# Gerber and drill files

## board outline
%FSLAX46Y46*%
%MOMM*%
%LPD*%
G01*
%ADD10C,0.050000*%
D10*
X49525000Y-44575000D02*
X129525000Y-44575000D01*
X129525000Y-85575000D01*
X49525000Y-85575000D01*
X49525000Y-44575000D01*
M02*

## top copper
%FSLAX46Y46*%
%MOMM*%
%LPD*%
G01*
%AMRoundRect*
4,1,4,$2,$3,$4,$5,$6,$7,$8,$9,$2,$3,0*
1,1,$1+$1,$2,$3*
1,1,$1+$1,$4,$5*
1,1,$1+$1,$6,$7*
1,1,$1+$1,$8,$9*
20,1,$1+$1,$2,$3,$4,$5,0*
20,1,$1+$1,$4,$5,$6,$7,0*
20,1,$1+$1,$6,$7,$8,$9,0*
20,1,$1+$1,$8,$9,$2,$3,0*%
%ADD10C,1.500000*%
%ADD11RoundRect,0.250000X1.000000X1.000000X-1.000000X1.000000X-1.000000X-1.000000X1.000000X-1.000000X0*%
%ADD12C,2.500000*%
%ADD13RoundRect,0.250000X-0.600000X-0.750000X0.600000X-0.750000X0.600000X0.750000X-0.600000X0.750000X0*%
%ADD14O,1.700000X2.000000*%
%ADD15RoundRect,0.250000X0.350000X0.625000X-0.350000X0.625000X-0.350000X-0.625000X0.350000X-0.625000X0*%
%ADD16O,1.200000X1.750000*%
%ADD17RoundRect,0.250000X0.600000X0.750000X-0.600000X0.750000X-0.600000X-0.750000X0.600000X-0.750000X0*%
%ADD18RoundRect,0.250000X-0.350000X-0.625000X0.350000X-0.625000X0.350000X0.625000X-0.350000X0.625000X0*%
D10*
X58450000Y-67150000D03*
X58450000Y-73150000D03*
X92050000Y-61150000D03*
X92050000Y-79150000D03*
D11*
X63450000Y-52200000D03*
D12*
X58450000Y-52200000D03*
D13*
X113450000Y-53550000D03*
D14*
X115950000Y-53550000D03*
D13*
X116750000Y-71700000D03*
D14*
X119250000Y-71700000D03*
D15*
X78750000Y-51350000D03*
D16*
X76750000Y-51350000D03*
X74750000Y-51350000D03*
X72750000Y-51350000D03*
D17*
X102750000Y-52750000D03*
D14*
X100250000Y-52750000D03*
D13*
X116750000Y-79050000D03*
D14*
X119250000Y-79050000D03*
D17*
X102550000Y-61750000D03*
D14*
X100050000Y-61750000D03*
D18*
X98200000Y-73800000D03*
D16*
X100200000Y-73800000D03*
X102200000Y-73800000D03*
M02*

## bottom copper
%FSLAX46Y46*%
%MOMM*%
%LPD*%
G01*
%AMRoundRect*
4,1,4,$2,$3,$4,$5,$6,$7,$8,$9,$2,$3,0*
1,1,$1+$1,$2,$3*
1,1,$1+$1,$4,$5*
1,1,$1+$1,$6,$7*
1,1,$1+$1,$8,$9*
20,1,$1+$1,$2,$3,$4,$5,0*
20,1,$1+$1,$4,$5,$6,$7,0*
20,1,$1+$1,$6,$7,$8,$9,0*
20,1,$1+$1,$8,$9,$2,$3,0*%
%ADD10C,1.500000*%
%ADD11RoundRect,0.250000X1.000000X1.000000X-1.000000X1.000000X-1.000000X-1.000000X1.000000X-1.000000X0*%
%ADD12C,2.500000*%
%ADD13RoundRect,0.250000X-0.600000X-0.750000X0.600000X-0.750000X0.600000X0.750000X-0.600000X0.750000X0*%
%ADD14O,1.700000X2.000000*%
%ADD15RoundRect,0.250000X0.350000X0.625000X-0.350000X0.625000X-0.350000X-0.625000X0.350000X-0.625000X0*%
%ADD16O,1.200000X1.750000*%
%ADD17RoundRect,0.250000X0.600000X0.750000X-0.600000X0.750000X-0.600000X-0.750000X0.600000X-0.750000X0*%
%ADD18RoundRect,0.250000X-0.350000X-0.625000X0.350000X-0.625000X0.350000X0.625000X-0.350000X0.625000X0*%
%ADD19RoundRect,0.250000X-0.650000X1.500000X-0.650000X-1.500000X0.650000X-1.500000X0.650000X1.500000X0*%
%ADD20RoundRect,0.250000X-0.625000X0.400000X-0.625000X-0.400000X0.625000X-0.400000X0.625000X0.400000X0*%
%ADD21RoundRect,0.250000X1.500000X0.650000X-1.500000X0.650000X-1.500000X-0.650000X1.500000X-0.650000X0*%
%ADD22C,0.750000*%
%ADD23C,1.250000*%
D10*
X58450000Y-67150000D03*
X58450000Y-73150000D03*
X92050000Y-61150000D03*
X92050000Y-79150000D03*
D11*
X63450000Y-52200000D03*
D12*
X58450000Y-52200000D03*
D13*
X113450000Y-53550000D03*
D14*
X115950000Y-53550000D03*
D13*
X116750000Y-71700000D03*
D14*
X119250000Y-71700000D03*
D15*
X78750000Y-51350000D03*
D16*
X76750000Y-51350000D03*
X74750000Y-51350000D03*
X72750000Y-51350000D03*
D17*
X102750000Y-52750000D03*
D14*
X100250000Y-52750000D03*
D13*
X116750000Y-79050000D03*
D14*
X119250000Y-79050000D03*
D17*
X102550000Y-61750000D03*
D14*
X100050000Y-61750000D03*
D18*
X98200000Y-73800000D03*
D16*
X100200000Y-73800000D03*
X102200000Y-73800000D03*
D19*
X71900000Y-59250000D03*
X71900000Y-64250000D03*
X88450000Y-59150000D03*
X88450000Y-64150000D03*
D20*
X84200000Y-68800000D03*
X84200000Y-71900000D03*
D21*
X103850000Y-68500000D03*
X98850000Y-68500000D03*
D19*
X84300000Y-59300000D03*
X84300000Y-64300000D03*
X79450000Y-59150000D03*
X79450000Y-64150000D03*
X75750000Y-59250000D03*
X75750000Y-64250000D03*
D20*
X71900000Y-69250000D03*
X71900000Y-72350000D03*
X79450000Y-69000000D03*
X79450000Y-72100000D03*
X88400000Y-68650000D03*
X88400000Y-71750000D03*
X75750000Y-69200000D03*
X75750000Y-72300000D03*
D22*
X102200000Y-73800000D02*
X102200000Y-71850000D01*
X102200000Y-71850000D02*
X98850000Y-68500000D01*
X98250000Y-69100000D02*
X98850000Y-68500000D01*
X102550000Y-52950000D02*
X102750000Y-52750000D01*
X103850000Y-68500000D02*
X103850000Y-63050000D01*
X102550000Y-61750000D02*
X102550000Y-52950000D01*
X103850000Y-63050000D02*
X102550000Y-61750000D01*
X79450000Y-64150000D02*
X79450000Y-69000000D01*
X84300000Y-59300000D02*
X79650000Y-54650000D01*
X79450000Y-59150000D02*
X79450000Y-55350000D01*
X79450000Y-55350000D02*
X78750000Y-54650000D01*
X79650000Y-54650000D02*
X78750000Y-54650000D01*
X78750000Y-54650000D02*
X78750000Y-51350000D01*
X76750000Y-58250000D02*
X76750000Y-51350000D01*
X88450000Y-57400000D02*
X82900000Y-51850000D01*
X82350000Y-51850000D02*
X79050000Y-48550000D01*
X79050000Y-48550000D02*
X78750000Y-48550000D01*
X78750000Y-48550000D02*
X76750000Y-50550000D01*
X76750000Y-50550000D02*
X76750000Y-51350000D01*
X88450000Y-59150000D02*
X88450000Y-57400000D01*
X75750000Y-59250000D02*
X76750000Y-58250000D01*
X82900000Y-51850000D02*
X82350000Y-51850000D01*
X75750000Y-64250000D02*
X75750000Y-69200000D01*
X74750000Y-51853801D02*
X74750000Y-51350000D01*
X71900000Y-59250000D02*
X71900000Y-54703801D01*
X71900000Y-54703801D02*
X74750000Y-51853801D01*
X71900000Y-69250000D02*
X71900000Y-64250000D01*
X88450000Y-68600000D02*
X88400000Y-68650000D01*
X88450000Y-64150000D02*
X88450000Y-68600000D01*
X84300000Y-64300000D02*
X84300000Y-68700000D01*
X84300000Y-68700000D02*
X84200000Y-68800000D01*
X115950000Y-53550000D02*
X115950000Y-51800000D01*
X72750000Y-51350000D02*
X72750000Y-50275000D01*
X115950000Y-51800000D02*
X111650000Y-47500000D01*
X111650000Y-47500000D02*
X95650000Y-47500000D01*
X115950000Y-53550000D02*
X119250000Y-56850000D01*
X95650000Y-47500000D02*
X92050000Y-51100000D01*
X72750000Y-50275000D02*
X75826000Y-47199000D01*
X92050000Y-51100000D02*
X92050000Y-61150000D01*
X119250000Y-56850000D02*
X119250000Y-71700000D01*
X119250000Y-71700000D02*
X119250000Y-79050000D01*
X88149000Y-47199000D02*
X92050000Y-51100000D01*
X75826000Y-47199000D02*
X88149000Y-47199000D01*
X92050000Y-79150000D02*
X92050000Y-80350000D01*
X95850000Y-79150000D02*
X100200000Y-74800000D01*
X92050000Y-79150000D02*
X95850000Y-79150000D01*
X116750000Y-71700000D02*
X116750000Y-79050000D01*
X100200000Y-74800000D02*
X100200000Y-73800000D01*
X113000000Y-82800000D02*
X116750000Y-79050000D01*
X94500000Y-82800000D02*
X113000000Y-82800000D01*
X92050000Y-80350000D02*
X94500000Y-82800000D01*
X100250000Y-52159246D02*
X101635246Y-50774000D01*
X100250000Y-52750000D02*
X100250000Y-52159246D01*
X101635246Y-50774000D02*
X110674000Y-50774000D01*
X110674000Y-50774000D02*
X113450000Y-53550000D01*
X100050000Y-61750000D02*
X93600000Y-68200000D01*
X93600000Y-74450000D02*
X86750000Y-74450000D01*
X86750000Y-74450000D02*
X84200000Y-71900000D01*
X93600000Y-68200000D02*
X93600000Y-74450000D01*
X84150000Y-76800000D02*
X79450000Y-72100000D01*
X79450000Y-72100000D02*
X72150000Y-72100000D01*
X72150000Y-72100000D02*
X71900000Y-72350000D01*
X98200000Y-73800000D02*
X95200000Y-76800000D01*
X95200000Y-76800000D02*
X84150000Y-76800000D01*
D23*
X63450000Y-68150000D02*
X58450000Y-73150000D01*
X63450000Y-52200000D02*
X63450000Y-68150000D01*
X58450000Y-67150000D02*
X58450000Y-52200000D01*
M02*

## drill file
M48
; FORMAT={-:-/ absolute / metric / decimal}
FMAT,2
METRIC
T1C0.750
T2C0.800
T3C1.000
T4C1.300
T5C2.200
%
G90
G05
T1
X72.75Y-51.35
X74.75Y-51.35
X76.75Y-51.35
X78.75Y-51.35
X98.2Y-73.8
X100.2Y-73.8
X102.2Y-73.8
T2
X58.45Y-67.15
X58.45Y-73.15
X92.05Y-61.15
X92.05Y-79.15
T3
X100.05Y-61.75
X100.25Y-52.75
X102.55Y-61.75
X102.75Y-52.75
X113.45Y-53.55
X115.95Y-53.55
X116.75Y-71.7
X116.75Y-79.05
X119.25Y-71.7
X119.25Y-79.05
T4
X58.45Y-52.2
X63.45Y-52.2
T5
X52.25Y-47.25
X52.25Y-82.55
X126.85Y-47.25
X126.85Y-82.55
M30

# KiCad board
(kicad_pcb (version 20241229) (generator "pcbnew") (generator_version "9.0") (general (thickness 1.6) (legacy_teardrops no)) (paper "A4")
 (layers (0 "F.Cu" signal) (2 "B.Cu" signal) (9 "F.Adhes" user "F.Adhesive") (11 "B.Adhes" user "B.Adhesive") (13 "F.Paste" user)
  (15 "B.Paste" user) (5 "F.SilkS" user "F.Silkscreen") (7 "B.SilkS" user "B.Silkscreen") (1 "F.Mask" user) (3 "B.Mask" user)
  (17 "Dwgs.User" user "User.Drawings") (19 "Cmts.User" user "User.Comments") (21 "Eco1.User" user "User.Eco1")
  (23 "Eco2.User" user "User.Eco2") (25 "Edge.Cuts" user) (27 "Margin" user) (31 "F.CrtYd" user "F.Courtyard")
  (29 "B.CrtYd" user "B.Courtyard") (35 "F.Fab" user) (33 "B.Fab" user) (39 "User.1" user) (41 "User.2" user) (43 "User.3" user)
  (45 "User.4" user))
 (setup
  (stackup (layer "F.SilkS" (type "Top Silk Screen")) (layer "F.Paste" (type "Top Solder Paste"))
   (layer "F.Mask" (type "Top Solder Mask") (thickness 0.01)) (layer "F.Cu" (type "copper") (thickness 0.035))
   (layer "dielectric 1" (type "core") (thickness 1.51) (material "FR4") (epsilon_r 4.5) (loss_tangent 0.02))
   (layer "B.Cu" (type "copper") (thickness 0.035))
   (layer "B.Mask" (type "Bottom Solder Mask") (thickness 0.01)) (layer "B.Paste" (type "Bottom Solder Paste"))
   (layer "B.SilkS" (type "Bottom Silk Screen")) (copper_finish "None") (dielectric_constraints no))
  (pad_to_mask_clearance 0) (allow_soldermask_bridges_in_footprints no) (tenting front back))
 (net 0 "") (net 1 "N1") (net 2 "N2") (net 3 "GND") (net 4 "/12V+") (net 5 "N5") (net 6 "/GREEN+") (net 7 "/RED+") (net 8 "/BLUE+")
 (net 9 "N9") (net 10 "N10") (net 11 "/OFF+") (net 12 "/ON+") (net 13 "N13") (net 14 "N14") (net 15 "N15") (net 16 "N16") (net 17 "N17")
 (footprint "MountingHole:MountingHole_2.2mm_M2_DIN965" (layer "F.Cu") (at 52.25 47.25)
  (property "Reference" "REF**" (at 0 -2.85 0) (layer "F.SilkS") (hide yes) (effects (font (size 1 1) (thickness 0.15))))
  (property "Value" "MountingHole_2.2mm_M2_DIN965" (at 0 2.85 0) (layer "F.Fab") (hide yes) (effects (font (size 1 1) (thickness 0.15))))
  (pad "" np_thru_hole circle (at 0 0) (size 2.2 2.2) (drill 2.2) (layers "*.Cu" "*.Mask")))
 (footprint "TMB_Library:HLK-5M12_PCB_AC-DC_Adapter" (layer "F.Cu") (at 75.25 70.15)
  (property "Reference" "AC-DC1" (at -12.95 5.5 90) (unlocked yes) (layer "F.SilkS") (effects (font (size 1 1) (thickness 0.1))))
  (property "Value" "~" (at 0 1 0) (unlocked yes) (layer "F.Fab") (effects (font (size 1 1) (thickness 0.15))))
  (pad "1" thru_hole circle (at -16.8 -3) (size 1.5 1.5) (drill 0.8) (layers "*.Cu" "*.Mask") (remove_unused_layers yes)
   (keep_end_layers yes) (zone_layer_connections) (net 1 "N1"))
  (pad "2" thru_hole circle (at -16.8 3) (size 1.5 1.5) (drill 0.8) (layers "*.Cu" "*.Mask") (remove_unused_layers yes)
   (keep_end_layers yes) (zone_layer_connections) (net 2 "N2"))
  (pad "3" thru_hole circle (at 16.8 -9) (size 1.5 1.5) (drill 0.8) (layers "*.Cu" "*.Mask") (remove_unused_layers yes)
   (keep_end_layers yes) (zone_layer_connections) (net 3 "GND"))
  (pad "4" thru_hole circle (at 16.8 9) (size 1.5 1.5) (drill 0.8) (layers "*.Cu" "*.Mask") (remove_unused_layers yes) (keep_end_layers yes)
   (zone_layer_connections) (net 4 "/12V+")))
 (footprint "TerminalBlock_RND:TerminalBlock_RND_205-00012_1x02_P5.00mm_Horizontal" (layer "F.Cu") (at 63.45 52.2 180)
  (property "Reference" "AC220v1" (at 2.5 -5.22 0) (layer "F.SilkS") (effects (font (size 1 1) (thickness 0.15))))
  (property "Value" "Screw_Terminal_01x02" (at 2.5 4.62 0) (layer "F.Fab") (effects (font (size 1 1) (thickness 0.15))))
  (pad "1" thru_hole roundrect (at 0 0 180) (size 2.5 2.5) (drill 1.3) (layers "*.Cu" "*.Mask") (remove_unused_layers no)
   (roundrect_rratio 0.1) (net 2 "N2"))
  (pad "2" thru_hole circle (at 5 0 180) (size 2.5 2.5) (drill 1.3) (layers "*.Cu" "*.Mask") (remove_unused_layers no) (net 1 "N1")))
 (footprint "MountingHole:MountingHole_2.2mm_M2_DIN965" (layer "F.Cu") (at 52.25 82.55)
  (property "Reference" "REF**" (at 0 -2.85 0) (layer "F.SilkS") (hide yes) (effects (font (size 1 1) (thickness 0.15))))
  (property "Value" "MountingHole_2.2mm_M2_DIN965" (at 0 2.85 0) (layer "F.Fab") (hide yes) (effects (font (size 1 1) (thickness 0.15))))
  (pad "" np_thru_hole circle (at 0 0) (size 2.2 2.2) (drill 2.2) (layers "*.Cu" "*.Mask")))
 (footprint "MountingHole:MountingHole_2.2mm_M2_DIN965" (layer "F.Cu") (at 126.85 82.55)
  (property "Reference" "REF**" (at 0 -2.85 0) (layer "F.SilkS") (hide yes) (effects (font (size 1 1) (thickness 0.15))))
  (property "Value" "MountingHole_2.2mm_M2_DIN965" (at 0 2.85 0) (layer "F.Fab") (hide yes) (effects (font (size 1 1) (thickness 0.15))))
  (pad "" np_thru_hole circle (at 0 0) (size 2.2 2.2) (drill 2.2) (layers "*.Cu" "*.Mask")))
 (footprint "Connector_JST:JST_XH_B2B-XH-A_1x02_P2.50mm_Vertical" (layer "F.Cu") (at 113.45 53.55)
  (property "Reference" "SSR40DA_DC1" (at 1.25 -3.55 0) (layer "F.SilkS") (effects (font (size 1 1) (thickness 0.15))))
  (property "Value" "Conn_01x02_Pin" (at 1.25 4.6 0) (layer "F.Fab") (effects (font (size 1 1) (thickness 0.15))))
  (pad "1" thru_hole roundrect (at 0 0) (size 1.7 2) (drill 1) (layers "*.Cu" "*.Mask") (remove_unused_layers no)
   (roundrect_rratio 0.147059) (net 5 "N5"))
  (pad "2" thru_hole oval (at 2.5 0) (size 1.7 2) (drill 1) (layers "*.Cu" "*.Mask") (remove_unused_layers no) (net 3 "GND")))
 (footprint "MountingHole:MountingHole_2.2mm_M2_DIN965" (layer "F.Cu") (at 126.85 47.25)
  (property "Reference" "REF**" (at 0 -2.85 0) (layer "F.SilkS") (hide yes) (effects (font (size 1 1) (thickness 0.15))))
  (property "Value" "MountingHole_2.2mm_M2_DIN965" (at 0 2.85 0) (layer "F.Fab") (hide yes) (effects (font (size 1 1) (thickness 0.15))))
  (pad "" np_thru_hole circle (at 0 0) (size 2.2 2.2) (drill 2.2) (layers "*.Cu" "*.Mask")))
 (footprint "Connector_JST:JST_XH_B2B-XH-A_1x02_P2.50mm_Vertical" (layer "F.Cu") (at 116.75 71.7)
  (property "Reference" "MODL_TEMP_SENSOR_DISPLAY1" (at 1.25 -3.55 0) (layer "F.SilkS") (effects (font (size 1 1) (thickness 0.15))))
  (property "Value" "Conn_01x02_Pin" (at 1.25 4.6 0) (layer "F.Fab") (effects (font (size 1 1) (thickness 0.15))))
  (pad "1" thru_hole roundrect (at 0 0) (size 1.7 2) (drill 1) (layers "*.Cu" "*.Mask") (remove_unused_layers no)
   (roundrect_rratio 0.147059) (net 4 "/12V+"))
  (pad "2" thru_hole oval (at 2.5 0) (size 1.7 2) (drill 1) (layers "*.Cu" "*.Mask") (remove_unused_layers no) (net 3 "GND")))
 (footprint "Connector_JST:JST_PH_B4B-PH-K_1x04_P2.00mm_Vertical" (layer "F.Cu") (at 78.75 51.35 180)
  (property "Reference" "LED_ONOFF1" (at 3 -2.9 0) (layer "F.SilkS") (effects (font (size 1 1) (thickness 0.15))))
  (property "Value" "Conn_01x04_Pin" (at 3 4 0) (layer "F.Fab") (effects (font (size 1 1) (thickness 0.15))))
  (pad "1" thru_hole roundrect (at 0 0 180) (size 1.2 1.75) (drill 0.75) (layers "*.Cu" "*.Mask") (remove_unused_layers no)
   (roundrect_rratio 0.208333) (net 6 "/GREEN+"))
  (pad "2" thru_hole oval (at 2 0 180) (size 1.2 1.75) (drill 0.75) (layers "*.Cu" "*.Mask") (remove_unused_layers no) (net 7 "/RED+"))
  (pad "3" thru_hole oval (at 4 0 180) (size 1.2 1.75) (drill 0.75) (layers "*.Cu" "*.Mask") (remove_unused_layers no) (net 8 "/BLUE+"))
  (pad "4" thru_hole oval (at 6 0 180) (size 1.2 1.75) (drill 0.75) (layers "*.Cu" "*.Mask") (remove_unused_layers no) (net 3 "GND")))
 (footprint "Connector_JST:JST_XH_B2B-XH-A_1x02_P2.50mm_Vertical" (layer "F.Cu") (at 102.75 52.75 180)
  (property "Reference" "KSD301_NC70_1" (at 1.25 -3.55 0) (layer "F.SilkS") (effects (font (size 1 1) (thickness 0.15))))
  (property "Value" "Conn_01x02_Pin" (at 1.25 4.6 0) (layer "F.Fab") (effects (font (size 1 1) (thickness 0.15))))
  (pad "1" thru_hole roundrect (at 0 0 180) (size 1.7 2) (drill 1) (layers "*.Cu" "*.Mask") (remove_unused_layers no)
   (roundrect_rratio 0.147059) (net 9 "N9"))
  (pad "2" thru_hole oval (at 2.5 0 180) (size 1.7 2) (drill 1) (layers "*.Cu" "*.Mask") (remove_unused_layers no) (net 5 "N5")))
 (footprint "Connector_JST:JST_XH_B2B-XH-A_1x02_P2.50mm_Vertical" (layer "F.Cu") (at 116.75 79.05)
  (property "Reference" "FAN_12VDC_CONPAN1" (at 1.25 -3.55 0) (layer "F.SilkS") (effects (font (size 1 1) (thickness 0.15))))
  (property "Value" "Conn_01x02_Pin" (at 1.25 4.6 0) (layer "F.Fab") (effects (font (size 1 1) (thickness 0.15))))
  (pad "1" thru_hole roundrect (at 0 0) (size 1.7 2) (drill 1) (layers "*.Cu" "*.Mask") (remove_unused_layers no)
   (roundrect_rratio 0.147059) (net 4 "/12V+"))
  (pad "2" thru_hole oval (at 2.5 0) (size 1.7 2) (drill 1) (layers "*.Cu" "*.Mask") (remove_unused_layers no) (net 3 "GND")))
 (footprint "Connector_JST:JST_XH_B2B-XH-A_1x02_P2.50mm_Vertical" (layer "F.Cu") (at 102.55 61.75 180)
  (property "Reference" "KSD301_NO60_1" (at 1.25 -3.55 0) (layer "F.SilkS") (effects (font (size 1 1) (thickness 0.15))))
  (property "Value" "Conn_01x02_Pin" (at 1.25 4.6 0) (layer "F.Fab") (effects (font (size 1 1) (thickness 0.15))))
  (pad "1" thru_hole roundrect (at 0 0 180) (size 1.7 2) (drill 1) (layers "*.Cu" "*.Mask") (remove_unused_layers no)
   (roundrect_rratio 0.147059) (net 9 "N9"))
  (pad "2" thru_hole oval (at 2.5 0 180) (size 1.7 2) (drill 1) (layers "*.Cu" "*.Mask") (remove_unused_layers no) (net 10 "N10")))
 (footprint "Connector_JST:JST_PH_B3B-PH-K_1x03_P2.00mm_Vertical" (layer "F.Cu") (at 98.2 73.8)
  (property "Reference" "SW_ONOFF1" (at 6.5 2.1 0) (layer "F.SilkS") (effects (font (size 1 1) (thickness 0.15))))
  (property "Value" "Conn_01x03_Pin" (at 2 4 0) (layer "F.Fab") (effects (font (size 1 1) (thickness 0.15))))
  (pad "1" thru_hole roundrect (at 0 0) (size 1.2 1.75) (drill 0.75) (layers "*.Cu" "*.Mask") (remove_unused_layers no)
   (roundrect_rratio 0.208333) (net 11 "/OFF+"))
  (pad "2" thru_hole oval (at 2 0) (size 1.2 1.75) (drill 0.75) (layers "*.Cu" "*.Mask") (remove_unused_layers no) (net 4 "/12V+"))
  (pad "3" thru_hole oval (at 4 0) (size 1.2 1.75) (drill 0.75) (layers "*.Cu" "*.Mask") (remove_unused_layers no) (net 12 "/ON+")))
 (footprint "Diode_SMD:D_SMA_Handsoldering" (layer "B.Cu") (at 71.9 61.75 -90)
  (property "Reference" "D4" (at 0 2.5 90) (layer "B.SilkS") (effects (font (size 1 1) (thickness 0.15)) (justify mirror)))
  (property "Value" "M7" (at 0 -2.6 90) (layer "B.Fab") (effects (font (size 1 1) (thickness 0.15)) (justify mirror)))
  (pad "1" smd roundrect (at -2.5 0 270) (size 3.5 1.8) (layers "B.Cu" "B.Mask" "B.Paste") (roundrect_rratio 0.1388888889) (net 8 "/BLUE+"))
  (pad "2" smd roundrect (at 2.5 0 270) (size 3.5 1.8) (layers "B.Cu" "B.Mask" "B.Paste") (roundrect_rratio 0.1388888889) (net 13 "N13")))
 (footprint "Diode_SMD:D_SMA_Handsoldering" (layer "B.Cu") (at 88.45 61.65 -90)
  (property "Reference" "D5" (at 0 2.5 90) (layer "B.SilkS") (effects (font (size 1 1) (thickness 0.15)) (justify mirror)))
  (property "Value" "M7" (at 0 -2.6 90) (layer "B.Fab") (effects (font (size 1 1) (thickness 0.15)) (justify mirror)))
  (pad "1" smd roundrect (at -2.5 0 270) (size 3.5 1.8) (layers "B.Cu" "B.Mask" "B.Paste") (roundrect_rratio 0.1388888889) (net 7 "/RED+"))
  (pad "2" smd roundrect (at 2.5 0 270) (size 3.5 1.8) (layers "B.Cu" "B.Mask" "B.Paste") (roundrect_rratio 0.1388888889) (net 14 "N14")))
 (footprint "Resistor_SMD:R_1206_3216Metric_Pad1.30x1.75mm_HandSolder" (layer "B.Cu") (at 84.2 70.35 -90)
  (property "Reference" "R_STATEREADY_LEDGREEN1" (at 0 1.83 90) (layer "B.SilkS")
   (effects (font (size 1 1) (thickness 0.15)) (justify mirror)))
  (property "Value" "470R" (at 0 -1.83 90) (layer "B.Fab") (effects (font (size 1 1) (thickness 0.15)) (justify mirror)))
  (pad "1" smd roundrect (at -1.55 0 270) (size 1.3 1.75) (layers "B.Cu" "B.Mask" "B.Paste") (roundrect_rratio 0.192308) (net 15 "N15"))
  (pad "2" smd roundrect (at 1.55 0 270) (size 1.3 1.75) (layers "B.Cu" "B.Mask" "B.Paste") (roundrect_rratio 0.192308) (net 10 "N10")))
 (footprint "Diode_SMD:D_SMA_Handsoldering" (layer "B.Cu") (at 101.35 68.5 180)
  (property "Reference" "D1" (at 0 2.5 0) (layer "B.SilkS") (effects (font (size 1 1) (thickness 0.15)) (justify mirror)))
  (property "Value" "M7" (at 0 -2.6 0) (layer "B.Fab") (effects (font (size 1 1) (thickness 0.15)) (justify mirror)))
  (pad "1" smd roundrect (at -2.5 0 180) (size 3.5 1.8) (layers "B.Cu" "B.Mask" "B.Paste") (roundrect_rratio 0.1388888889) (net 9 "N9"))
  (pad "2" smd roundrect (at 2.5 0 180) (size 3.5 1.8) (layers "B.Cu" "B.Mask" "B.Paste") (roundrect_rratio 0.1388888889) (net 12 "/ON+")))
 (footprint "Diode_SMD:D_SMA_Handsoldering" (layer "B.Cu") (at 84.3 61.8 -90)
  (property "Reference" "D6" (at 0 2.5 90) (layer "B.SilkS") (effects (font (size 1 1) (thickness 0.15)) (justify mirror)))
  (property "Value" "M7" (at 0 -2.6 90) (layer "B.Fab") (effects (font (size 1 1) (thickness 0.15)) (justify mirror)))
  (pad "1" smd roundrect (at -2.5 0 270) (size 3.5 1.8) (layers "B.Cu" "B.Mask" "B.Paste") (roundrect_rratio 0.1388888889) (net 6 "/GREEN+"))
  (pad "2" smd roundrect (at 2.5 0 270) (size 3.5 1.8) (layers "B.Cu" "B.Mask" "B.Paste") (roundrect_rratio 0.1388888889) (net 15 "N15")))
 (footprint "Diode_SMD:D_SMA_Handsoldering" (layer "B.Cu") (at 79.45 61.65 -90)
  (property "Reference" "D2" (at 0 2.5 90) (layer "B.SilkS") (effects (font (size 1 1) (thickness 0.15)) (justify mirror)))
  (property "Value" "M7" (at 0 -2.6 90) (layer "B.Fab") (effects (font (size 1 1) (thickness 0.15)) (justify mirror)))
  (pad "1" smd roundrect (at -2.5 0 270) (size 3.5 1.8) (layers "B.Cu" "B.Mask" "B.Paste") (roundrect_rratio 0.1388888889) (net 6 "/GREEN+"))
  (pad "2" smd roundrect (at 2.5 0 270) (size 3.5 1.8) (layers "B.Cu" "B.Mask" "B.Paste") (roundrect_rratio 0.1388888889) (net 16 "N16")))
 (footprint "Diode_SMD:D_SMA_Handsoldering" (layer "B.Cu") (at 75.75 61.75 -90)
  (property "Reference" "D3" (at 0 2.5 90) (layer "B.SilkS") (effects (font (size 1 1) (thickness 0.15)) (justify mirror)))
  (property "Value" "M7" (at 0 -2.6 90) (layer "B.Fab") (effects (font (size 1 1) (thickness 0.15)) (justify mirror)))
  (pad "1" smd roundrect (at -2.5 0 270) (size 3.5 1.8) (layers "B.Cu" "B.Mask" "B.Paste") (roundrect_rratio 0.1388888889) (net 7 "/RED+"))
  (pad "2" smd roundrect (at 2.5 0 270) (size 3.5 1.8) (layers "B.Cu" "B.Mask" "B.Paste") (roundrect_rratio 0.1388888889) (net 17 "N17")))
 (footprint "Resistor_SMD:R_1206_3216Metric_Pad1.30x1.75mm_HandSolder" (layer "B.Cu") (at 71.9 70.8 -90)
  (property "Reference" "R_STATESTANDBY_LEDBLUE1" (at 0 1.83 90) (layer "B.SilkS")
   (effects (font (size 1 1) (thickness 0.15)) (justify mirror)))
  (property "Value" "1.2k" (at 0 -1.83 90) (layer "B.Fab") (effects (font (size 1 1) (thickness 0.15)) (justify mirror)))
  (pad "1" smd roundrect (at -1.55 0 270) (size 1.3 1.75) (layers "B.Cu" "B.Mask" "B.Paste") (roundrect_rratio 0.192308) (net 13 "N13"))
  (pad "2" smd roundrect (at 1.55 0 270) (size 1.3 1.75) (layers "B.Cu" "B.Mask" "B.Paste") (roundrect_rratio 0.192308) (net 11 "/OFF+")))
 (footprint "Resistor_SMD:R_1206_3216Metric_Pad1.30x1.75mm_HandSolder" (layer "B.Cu") (at 79.45 70.55 -90)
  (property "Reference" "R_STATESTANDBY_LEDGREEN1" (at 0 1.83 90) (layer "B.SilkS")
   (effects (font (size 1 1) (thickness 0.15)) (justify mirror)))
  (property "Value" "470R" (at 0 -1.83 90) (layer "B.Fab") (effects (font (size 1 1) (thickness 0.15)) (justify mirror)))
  (pad "1" smd roundrect (at -1.55 0 270) (size 1.3 1.75) (layers "B.Cu" "B.Mask" "B.Paste") (roundrect_rratio 0.192308) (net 16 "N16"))
  (pad "2" smd roundrect (at 1.55 0 270) (size 1.3 1.75) (layers "B.Cu" "B.Mask" "B.Paste") (roundrect_rratio 0.192308) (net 11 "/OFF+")))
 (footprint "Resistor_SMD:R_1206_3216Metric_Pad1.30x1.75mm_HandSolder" (layer "B.Cu") (at 88.4 70.2 -90)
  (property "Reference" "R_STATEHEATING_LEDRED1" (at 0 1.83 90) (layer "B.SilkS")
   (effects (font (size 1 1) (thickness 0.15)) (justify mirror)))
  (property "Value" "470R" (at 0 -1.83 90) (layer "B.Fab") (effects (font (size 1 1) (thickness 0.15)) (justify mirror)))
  (pad "1" smd roundrect (at -1.55 0 270) (size 1.3 1.75) (layers "B.Cu" "B.Mask" "B.Paste") (roundrect_rratio 0.192308) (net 14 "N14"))
  (pad "2" smd roundrect (at 1.55 0 270) (size 1.3 1.75) (layers "B.Cu" "B.Mask" "B.Paste") (roundrect_rratio 0.192308) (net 5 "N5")))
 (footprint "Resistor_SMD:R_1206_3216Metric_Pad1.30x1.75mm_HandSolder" (layer "B.Cu") (at 75.75 70.75 -90)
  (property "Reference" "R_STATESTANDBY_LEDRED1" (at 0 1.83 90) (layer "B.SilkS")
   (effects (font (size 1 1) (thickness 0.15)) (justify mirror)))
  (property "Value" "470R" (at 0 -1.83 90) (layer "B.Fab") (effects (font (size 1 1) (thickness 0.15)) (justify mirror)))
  (pad "1" smd roundrect (at -1.55 0 270) (size 1.3 1.75) (layers "B.Cu" "B.Mask" "B.Paste") (roundrect_rratio 0.192308) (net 17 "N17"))
  (pad "2" smd roundrect (at 1.55 0 270) (size 1.3 1.75) (layers "B.Cu" "B.Mask" "B.Paste") (roundrect_rratio 0.192308) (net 11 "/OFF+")))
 (gr_rect (start 49.525 44.575) (end 129.525 85.575) (stroke (width 0.05) (type solid)) (fill no) (layer "Edge.Cuts"))
 (segment (start 102.2 73.8) (end 102.2 71.85) (width 0.75) (layer "B.Cu") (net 12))
 (segment (start 102.2 71.85) (end 98.85 68.5) (width 0.75) (layer "B.Cu") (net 12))
 (segment (start 98.25 69.1) (end 98.85 68.5) (width 0.75) (layer "B.Cu") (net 12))
 (segment (start 102.55 52.95) (end 102.75 52.75) (width 0.75) (layer "B.Cu") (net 9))
 (segment (start 103.85 68.5) (end 103.85 63.05) (width 0.75) (layer "B.Cu") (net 9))
 (segment (start 102.55 61.75) (end 102.55 52.95) (width 0.75) (layer "B.Cu") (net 9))
 (segment (start 103.85 63.05) (end 102.55 61.75) (width 0.75) (layer "B.Cu") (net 9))
 (segment (start 79.45 64.15) (end 79.45 69) (width 0.75) (layer "B.Cu") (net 16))
 (segment (start 84.3 59.3) (end 79.65 54.65) (width 0.75) (layer "B.Cu") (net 6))
 (segment (start 79.45 59.15) (end 79.45 55.35) (width 0.75) (layer "B.Cu") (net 6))
 (segment (start 79.45 55.35) (end 78.75 54.65) (width 0.75) (layer "B.Cu") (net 6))
 (segment (start 79.65 54.65) (end 78.75 54.65) (width 0.75) (layer "B.Cu") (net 6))
 (segment (start 78.75 54.65) (end 78.75 51.35) (width 0.75) (layer "B.Cu") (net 6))
 (segment (start 76.75 58.25) (end 76.75 51.35) (width 0.75) (layer "B.Cu") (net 7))
 (segment (start 88.45 57.4) (end 82.9 51.85) (width 0.75) (layer "B.Cu") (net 7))
 (segment (start 82.35 51.85) (end 79.05 48.55) (width 0.75) (layer "B.Cu") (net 7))
 (segment (start 79.05 48.55) (end 78.75 48.55) (width 0.75) (layer "B.Cu") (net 7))
 (segment (start 78.75 48.55) (end 76.75 50.55) (width 0.75) (layer "B.Cu") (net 7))
 (segment (start 76.75 50.55) (end 76.75 51.35) (width 0.75) (layer "B.Cu") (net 7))
 (segment (start 88.45 59.15) (end 88.45 57.4) (width 0.75) (layer "B.Cu") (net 7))
 (segment (start 75.75 59.25) (end 76.75 58.25) (width 0.75) (layer "B.Cu") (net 7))
 (segment (start 82.9 51.85) (end 82.35 51.85) (width 0.75) (layer "B.Cu") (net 7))
 (segment (start 75.75 64.25) (end 75.75 69.2) (width 0.75) (layer "B.Cu") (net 17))
 (segment (start 74.75 51.853801) (end 74.75 51.35) (width 0.75) (layer "B.Cu") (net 8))
 (segment (start 71.9 59.25) (end 71.9 54.703801) (width 0.75) (layer "B.Cu") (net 8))
 (segment (start 71.9 54.703801) (end 74.75 51.853801) (width 0.75) (layer "B.Cu") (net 8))
 (segment (start 71.9 69.25) (end 71.9 64.25) (width 0.75) (layer "B.Cu") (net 13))
 (segment (start 88.45 68.6) (end 88.4 68.65) (width 0.75) (layer "B.Cu") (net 14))
 (segment (start 88.45 64.15) (end 88.45 68.6) (width 0.75) (layer "B.Cu") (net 14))
 (segment (start 84.3 64.3) (end 84.3 68.7) (width 0.75) (layer "B.Cu") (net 15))
 (segment (start 84.3 68.7) (end 84.2 68.8) (width 0.75) (layer "B.Cu") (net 15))
 (segment (start 115.95 53.55) (end 115.95 51.8) (width 0.75) (layer "B.Cu") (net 3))
 (segment (start 72.75 51.35) (end 72.75 50.275) (width 0.75) (layer "B.Cu") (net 3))
 (segment (start 115.95 51.8) (end 111.65 47.5) (width 0.75) (layer "B.Cu") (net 3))
 (segment (start 111.65 47.5) (end 95.65 47.5) (width 0.75) (layer "B.Cu") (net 3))
 (segment (start 115.95 53.55) (end 119.25 56.85) (width 0.75) (layer "B.Cu") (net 3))
 (segment (start 95.65 47.5) (end 92.05 51.1) (width 0.75) (layer "B.Cu") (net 3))
 (segment (start 72.75 50.275) (end 75.826 47.199) (width 0.75) (layer "B.Cu") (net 3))
 (segment (start 92.05 51.1) (end 92.05 61.15) (width 0.75) (layer "B.Cu") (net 3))
 (segment (start 119.25 56.85) (end 119.25 71.7) (width 0.75) (layer "B.Cu") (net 3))
 (segment (start 119.25 71.7) (end 119.25 79.05) (width 0.75) (layer "B.Cu") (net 3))
 (segment (start 88.149 47.199) (end 92.05 51.1) (width 0.75) (layer "B.Cu") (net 3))
 (segment (start 75.826 47.199) (end 88.149 47.199) (width 0.75) (layer "B.Cu") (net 3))
 (segment (start 92.05 79.15) (end 92.05 80.35) (width 0.75) (layer "B.Cu") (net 4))
 (segment (start 95.85 79.15) (end 100.2 74.8) (width 0.75) (layer "B.Cu") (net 4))
 (segment (start 92.05 79.15) (end 95.85 79.15) (width 0.75) (layer "B.Cu") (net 4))
 (segment (start 116.75 71.7) (end 116.75 79.05) (width 0.75) (layer "B.Cu") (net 4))
 (segment (start 100.2 74.8) (end 100.2 73.8) (width 0.75) (layer "B.Cu") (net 4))
 (segment (start 113 82.8) (end 116.75 79.05) (width 0.75) (layer "B.Cu") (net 4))
 (segment (start 94.5 82.8) (end 113 82.8) (width 0.75) (layer "B.Cu") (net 4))
 (segment (start 92.05 80.35) (end 94.5 82.8) (width 0.75) (layer "B.Cu") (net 4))
 (segment (start 100.25 52.159246) (end 101.635246 50.774) (width 0.75) (layer "B.Cu") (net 5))
 (segment (start 100.25 52.75) (end 100.25 52.159246) (width 0.75) (layer "B.Cu") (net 5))
 (segment (start 101.635246 50.774) (end 110.674 50.774) (width 0.75) (layer "B.Cu") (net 5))
 (segment (start 110.674 50.774) (end 113.45 53.55) (width 0.75) (layer "B.Cu") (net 5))
 (segment (start 100.05 61.75) (end 93.6 68.2) (width 0.75) (layer "B.Cu") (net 10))
 (segment (start 93.6 74.45) (end 86.75 74.45) (width 0.75) (layer "B.Cu") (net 10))
 (segment (start 86.75 74.45) (end 84.2 71.9) (width 0.75) (layer "B.Cu") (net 10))
 (segment (start 93.6 68.2) (end 93.6 74.45) (width 0.75) (layer "B.Cu") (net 10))
 (segment (start 84.15 76.8) (end 79.45 72.1) (width 0.75) (layer "B.Cu") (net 11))
 (segment (start 79.45 72.1) (end 72.15 72.1) (width 0.75) (layer "B.Cu") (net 11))
 (segment (start 72.15 72.1) (end 71.9 72.35) (width 0.75) (layer "B.Cu") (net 11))
 (segment (start 98.2 73.8) (end 95.2 76.8) (width 0.75) (layer "B.Cu") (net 11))
 (segment (start 95.2 76.8) (end 84.15 76.8) (width 0.75) (layer "B.Cu") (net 11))
 (segment (start 63.45 68.15) (end 58.45 73.15) (width 1.25) (layer "B.Cu") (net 2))
 (segment (start 63.45 52.2) (end 63.45 68.15) (width 1.25) (layer "B.Cu") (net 2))
 (segment (start 58.45 67.15) (end 58.45 52.2) (width 1.25) (layer "B.Cu") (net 1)))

